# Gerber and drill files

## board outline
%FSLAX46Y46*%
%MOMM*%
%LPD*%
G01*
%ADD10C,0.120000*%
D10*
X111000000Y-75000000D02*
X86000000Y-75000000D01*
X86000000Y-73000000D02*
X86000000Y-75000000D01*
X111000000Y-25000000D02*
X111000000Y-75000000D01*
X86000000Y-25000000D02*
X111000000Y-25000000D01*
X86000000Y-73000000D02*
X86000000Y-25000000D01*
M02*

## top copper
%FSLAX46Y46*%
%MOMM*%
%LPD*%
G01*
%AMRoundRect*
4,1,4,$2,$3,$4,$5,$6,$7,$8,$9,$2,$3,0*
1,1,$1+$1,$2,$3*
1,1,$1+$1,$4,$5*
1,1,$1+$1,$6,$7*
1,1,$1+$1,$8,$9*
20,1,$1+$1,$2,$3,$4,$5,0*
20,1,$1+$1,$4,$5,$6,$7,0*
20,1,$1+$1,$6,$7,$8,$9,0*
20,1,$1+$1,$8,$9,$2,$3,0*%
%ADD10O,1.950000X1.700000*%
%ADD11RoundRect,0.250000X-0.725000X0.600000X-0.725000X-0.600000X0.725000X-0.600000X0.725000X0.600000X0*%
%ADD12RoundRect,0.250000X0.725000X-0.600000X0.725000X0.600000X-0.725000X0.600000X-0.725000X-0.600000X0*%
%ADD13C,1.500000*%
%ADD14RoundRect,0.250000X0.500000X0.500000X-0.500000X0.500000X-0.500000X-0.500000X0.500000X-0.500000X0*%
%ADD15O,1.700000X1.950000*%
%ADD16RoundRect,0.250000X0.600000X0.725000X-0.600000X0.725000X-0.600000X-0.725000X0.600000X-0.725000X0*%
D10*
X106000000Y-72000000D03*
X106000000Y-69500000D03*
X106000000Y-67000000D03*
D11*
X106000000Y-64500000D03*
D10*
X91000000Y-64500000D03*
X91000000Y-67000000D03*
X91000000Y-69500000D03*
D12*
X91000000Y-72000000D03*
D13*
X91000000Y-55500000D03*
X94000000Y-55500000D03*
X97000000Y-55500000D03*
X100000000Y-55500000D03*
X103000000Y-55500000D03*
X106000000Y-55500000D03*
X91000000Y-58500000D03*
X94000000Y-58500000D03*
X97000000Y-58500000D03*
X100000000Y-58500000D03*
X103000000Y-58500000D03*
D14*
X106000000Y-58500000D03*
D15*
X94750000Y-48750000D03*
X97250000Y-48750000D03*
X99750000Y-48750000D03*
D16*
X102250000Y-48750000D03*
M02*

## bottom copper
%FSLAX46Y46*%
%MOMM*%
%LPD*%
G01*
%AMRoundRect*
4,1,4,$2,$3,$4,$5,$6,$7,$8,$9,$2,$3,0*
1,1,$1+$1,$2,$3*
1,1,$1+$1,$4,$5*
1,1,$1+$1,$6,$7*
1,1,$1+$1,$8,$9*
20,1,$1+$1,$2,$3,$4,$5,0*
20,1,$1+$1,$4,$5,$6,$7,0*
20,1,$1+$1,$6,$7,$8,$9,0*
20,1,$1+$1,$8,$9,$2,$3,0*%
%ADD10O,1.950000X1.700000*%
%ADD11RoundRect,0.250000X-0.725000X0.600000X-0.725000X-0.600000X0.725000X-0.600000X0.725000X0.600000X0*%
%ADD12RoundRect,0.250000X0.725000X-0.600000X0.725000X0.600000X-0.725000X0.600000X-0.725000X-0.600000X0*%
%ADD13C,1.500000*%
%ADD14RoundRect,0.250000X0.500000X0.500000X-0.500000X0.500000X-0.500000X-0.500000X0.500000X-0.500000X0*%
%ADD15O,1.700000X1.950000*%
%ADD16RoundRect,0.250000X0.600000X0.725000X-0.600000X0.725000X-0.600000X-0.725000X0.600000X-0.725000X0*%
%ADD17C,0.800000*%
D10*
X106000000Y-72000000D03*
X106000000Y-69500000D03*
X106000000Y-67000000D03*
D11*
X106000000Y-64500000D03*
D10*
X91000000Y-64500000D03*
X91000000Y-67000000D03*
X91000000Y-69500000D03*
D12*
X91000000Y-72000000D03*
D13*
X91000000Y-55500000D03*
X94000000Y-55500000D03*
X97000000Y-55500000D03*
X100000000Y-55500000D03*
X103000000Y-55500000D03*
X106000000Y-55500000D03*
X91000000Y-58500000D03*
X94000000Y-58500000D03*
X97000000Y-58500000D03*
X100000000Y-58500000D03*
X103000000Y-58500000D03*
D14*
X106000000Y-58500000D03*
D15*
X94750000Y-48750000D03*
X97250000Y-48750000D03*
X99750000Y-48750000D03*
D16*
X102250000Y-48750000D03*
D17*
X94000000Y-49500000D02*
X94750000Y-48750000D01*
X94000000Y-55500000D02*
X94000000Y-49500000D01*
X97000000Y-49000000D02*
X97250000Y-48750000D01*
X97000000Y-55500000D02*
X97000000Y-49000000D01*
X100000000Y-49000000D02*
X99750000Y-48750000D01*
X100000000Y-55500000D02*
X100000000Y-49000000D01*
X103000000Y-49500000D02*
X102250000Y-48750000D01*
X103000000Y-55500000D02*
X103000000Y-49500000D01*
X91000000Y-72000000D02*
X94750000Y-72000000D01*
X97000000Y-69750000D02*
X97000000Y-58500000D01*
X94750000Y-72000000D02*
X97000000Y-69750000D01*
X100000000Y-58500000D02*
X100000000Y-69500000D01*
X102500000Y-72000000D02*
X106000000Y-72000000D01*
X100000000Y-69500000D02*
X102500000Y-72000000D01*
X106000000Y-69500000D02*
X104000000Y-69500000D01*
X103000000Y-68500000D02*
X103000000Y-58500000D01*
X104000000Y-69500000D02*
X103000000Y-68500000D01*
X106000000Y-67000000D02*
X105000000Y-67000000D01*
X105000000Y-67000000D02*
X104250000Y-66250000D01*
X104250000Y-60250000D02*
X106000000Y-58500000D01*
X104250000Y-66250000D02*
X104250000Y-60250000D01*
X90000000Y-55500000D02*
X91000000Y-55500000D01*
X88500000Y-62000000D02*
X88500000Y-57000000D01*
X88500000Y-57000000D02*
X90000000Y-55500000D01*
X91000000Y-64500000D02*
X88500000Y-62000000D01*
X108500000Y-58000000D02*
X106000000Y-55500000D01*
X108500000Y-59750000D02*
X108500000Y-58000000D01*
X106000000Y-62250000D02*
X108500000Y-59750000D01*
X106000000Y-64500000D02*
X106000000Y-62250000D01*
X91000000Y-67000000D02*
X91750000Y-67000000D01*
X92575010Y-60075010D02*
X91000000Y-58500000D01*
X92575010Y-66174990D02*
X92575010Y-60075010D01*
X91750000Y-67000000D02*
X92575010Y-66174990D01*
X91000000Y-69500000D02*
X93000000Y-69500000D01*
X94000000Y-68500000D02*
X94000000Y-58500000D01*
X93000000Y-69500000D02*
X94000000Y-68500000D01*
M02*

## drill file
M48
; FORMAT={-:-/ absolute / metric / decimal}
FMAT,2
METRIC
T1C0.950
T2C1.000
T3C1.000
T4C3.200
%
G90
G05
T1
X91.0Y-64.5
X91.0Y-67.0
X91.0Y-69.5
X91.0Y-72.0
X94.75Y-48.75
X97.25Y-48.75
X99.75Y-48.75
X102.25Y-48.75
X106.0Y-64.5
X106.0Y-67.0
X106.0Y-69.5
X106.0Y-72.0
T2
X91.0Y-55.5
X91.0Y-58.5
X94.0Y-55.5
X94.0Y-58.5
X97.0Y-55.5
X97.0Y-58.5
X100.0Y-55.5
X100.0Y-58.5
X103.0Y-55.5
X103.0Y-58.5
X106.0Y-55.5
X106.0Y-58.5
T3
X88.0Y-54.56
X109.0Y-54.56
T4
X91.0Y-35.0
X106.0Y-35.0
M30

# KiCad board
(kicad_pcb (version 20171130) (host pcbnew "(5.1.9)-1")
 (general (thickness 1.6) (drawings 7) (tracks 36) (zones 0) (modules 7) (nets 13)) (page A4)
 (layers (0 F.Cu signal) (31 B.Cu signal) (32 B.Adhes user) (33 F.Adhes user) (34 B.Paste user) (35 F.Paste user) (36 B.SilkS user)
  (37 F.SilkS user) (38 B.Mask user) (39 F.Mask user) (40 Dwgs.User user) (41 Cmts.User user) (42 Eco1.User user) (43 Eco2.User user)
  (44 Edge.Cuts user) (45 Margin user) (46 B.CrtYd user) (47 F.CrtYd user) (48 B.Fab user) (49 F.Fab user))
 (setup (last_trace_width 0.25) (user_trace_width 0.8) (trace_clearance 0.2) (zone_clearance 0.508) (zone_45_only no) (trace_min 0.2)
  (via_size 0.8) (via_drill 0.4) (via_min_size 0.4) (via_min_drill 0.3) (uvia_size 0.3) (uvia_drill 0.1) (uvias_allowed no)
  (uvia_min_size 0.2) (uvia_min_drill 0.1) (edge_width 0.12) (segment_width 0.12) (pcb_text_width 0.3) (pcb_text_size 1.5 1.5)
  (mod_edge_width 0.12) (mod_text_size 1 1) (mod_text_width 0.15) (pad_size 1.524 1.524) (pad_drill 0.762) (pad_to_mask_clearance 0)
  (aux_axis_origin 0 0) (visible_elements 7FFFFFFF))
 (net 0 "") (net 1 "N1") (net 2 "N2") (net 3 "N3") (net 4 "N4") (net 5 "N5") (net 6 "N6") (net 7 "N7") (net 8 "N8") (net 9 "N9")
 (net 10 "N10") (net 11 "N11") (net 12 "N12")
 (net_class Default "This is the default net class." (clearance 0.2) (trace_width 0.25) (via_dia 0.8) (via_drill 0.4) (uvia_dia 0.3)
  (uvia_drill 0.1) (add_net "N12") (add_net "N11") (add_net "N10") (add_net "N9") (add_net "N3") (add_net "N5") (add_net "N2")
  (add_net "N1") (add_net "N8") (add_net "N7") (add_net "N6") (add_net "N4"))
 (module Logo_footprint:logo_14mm (layer F.Cu) (at 98.5 32)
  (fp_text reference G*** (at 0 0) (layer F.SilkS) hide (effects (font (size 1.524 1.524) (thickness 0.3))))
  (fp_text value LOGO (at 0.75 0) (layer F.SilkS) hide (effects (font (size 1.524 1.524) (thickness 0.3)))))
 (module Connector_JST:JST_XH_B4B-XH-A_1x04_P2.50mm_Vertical (layer F.Cu) (at 106 64.5 270)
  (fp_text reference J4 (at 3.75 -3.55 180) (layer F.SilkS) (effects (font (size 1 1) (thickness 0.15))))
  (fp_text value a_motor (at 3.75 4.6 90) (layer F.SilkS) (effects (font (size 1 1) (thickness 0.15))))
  (pad 4 thru_hole oval (at 7.5 0 270) (size 1.7 1.95) (drill 0.95) (layers *.Cu *.Mask) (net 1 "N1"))
  (pad 3 thru_hole oval (at 5 0 270) (size 1.7 1.95) (drill 0.95) (layers *.Cu *.Mask) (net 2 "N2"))
  (pad 2 thru_hole oval (at 2.5 0 270) (size 1.7 1.95) (drill 0.95) (layers *.Cu *.Mask) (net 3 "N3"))
  (pad 1 thru_hole roundrect (at 0 0 270) (size 1.7 1.95) (drill 0.95) (layers *.Cu *.Mask) (roundrect_rratio 0.1470588235294118)
   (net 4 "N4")))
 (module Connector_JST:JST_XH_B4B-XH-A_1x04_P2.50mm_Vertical (layer F.Cu) (at 91 72 90)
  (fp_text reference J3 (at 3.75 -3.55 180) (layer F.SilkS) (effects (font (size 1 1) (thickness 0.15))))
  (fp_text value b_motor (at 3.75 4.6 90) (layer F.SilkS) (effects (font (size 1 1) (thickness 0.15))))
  (pad 4 thru_hole oval (at 7.5 0 90) (size 1.7 1.95) (drill 0.95) (layers *.Cu *.Mask) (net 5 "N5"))
  (pad 3 thru_hole oval (at 5 0 90) (size 1.7 1.95) (drill 0.95) (layers *.Cu *.Mask) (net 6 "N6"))
  (pad 2 thru_hole oval (at 2.5 0 90) (size 1.7 1.95) (drill 0.95) (layers *.Cu *.Mask) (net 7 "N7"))
  (pad 1 thru_hole roundrect (at 0 0 90) (size 1.7 1.95) (drill 0.95) (layers *.Cu *.Mask) (roundrect_rratio 0.1470588235294118)
   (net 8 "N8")))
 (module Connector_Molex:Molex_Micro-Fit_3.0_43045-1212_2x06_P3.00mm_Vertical (layer F.Cu) (at 106 58.5 180)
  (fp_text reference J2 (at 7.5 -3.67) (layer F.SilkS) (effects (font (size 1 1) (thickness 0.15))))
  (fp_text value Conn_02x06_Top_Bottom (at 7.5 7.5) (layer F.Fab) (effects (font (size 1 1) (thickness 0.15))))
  (pad 12 thru_hole circle (at 15 3 180) (size 1.5 1.5) (drill 1) (layers *.Cu *.Mask) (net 5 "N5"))
  (pad 11 thru_hole circle (at 12 3 180) (size 1.5 1.5) (drill 1) (layers *.Cu *.Mask) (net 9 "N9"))
  (pad 10 thru_hole circle (at 9 3 180) (size 1.5 1.5) (drill 1) (layers *.Cu *.Mask) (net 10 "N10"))
  (pad 9 thru_hole circle (at 6 3 180) (size 1.5 1.5) (drill 1) (layers *.Cu *.Mask) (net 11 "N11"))
  (pad 8 thru_hole circle (at 3 3 180) (size 1.5 1.5) (drill 1) (layers *.Cu *.Mask) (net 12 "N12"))
  (pad 7 thru_hole circle (at 0 3 180) (size 1.5 1.5) (drill 1) (layers *.Cu *.Mask) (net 4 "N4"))
  (pad 6 thru_hole circle (at 15 0 180) (size 1.5 1.5) (drill 1) (layers *.Cu *.Mask) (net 6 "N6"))
  (pad 5 thru_hole circle (at 12 0 180) (size 1.5 1.5) (drill 1) (layers *.Cu *.Mask) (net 7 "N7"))
  (pad 4 thru_hole circle (at 9 0 180) (size 1.5 1.5) (drill 1) (layers *.Cu *.Mask) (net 8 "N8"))
  (pad 3 thru_hole circle (at 6 0 180) (size 1.5 1.5) (drill 1) (layers *.Cu *.Mask) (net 1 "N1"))
  (pad 2 thru_hole circle (at 3 0 180) (size 1.5 1.5) (drill 1) (layers *.Cu *.Mask) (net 2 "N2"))
  (pad 1 thru_hole roundrect (at 0 0 180) (size 1.5 1.5) (drill 1) (layers *.Cu *.Mask) (roundrect_rratio 0.1666666666666667) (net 3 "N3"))
  (pad "" np_thru_hole circle (at 18 3.94 180) (size 1 1) (drill 1) (layers *.Cu *.Mask))
  (pad "" np_thru_hole circle (at -3 3.94 180) (size 1 1) (drill 1) (layers *.Cu *.Mask)))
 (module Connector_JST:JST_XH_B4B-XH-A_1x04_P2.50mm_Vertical (layer F.Cu) (at 102.25 48.75 180)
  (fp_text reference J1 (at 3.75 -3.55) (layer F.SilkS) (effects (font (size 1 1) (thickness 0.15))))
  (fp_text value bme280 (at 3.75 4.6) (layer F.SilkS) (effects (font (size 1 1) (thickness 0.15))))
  (pad 4 thru_hole oval (at 7.5 0 180) (size 1.7 1.95) (drill 0.95) (layers *.Cu *.Mask) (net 9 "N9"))
  (pad 3 thru_hole oval (at 5 0 180) (size 1.7 1.95) (drill 0.95) (layers *.Cu *.Mask) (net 10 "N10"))
  (pad 2 thru_hole oval (at 2.5 0 180) (size 1.7 1.95) (drill 0.95) (layers *.Cu *.Mask) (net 11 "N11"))
  (pad 1 thru_hole roundrect (at 0 0 180) (size 1.7 1.95) (drill 0.95) (layers *.Cu *.Mask) (roundrect_rratio 0.1470588235294118)
   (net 12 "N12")))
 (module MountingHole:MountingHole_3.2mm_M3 (layer F.Cu) (at 106 35 180)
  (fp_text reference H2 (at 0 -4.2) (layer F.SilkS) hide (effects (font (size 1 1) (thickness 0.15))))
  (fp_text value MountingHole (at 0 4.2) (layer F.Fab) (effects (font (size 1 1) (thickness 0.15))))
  (pad 1 np_thru_hole circle (at 0 0 180) (size 3.2 3.2) (drill 3.2) (layers *.Cu *.Mask)))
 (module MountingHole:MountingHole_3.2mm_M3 (layer F.Cu) (at 91 35 180)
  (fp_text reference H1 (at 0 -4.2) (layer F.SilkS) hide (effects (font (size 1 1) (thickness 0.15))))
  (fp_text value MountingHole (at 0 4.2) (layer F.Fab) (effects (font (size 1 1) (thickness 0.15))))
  (pad 1 np_thru_hole circle (at 0 0 180) (size 3.2 3.2) (drill 3.2) (layers *.Cu *.Mask)))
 (gr_line (start 111 75) (end 86 75) (layer Edge.Cuts) (width 0.12))
 (gr_line (start 86 73) (end 86 75) (layer Edge.Cuts) (width 0.12))
 (gr_line (start 111 25) (end 111 75) (layer Edge.Cuts) (width 0.12))
 (gr_line (start 86 25) (end 111 25) (layer Edge.Cuts) (width 0.12))
 (gr_line (start 86 73) (end 86 25) (layer Edge.Cuts) (width 0.12))
 (segment (start 94 49.5) (end 94.75 48.75) (width 0.8) (layer B.Cu) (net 9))
 (segment (start 94 55.5) (end 94 49.5) (width 0.8) (layer B.Cu) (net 9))
 (segment (start 97 49) (end 97.25 48.75) (width 0.8) (layer B.Cu) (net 10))
 (segment (start 97 55.5) (end 97 49) (width 0.8) (layer B.Cu) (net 10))
 (segment (start 100 49) (end 99.75 48.75) (width 0.8) (layer B.Cu) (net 11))
 (segment (start 100 55.5) (end 100 49) (width 0.8) (layer B.Cu) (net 11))
 (segment (start 103 49.5) (end 102.25 48.75) (width 0.8) (layer B.Cu) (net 12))
 (segment (start 103 55.5) (end 103 49.5) (width 0.8) (layer B.Cu) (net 12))
 (segment (start 91 72) (end 94.75 72) (width 0.8) (layer B.Cu) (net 8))
 (segment (start 97 69.75) (end 97 58.5) (width 0.8) (layer B.Cu) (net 8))
 (segment (start 94.75 72) (end 97 69.75) (width 0.8) (layer B.Cu) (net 8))
 (segment (start 100 58.5) (end 100 69.5) (width 0.8) (layer B.Cu) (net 1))
 (segment (start 102.5 72) (end 106 72) (width 0.8) (layer B.Cu) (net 1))
 (segment (start 100 69.5) (end 102.5 72) (width 0.8) (layer B.Cu) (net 1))
 (segment (start 106 69.5) (end 104 69.5) (width 0.8) (layer B.Cu) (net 2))
 (segment (start 103 68.5) (end 103 58.5) (width 0.8) (layer B.Cu) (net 2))
 (segment (start 104 69.5) (end 103 68.5) (width 0.8) (layer B.Cu) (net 2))
 (segment (start 106 67) (end 105 67) (width 0.8) (layer B.Cu) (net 3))
 (segment (start 105 67) (end 104.25 66.25) (width 0.8) (layer B.Cu) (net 3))
 (segment (start 104.25 60.25) (end 106 58.5) (width 0.8) (layer B.Cu) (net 3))
 (segment (start 104.25 66.25) (end 104.25 60.25) (width 0.8) (layer B.Cu) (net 3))
 (segment (start 90 55.5) (end 91 55.5) (width 0.8) (layer B.Cu) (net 5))
 (segment (start 88.5 62) (end 88.5 57) (width 0.8) (layer B.Cu) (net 5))
 (segment (start 88.5 57) (end 90 55.5) (width 0.8) (layer B.Cu) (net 5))
 (segment (start 91 64.5) (end 88.5 62) (width 0.8) (layer B.Cu) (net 5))
 (segment (start 108.5 58) (end 106 55.5) (width 0.8) (layer B.Cu) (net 4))
 (segment (start 108.5 59.75) (end 108.5 58) (width 0.8) (layer B.Cu) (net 4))
 (segment (start 106 62.25) (end 108.5 59.75) (width 0.8) (layer B.Cu) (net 4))
 (segment (start 106 64.5) (end 106 62.25) (width 0.8) (layer B.Cu) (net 4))
 (segment (start 91 67) (end 91.75 67) (width 0.8) (layer B.Cu) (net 6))
 (segment (start 92.57501 60.07501) (end 91 58.5) (width 0.8) (layer B.Cu) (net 6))
 (segment (start 92.57501 66.17499) (end 92.57501 60.07501) (width 0.8) (layer B.Cu) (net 6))
 (segment (start 91.75 67) (end 92.57501 66.17499) (width 0.8) (layer B.Cu) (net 6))
 (segment (start 91 69.5) (end 93 69.5) (width 0.8) (layer B.Cu) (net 7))
 (segment (start 94 68.5) (end 94 58.5) (width 0.8) (layer B.Cu) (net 7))
 (segment (start 93 69.5) (end 94 68.5) (width 0.8) (layer B.Cu) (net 7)))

